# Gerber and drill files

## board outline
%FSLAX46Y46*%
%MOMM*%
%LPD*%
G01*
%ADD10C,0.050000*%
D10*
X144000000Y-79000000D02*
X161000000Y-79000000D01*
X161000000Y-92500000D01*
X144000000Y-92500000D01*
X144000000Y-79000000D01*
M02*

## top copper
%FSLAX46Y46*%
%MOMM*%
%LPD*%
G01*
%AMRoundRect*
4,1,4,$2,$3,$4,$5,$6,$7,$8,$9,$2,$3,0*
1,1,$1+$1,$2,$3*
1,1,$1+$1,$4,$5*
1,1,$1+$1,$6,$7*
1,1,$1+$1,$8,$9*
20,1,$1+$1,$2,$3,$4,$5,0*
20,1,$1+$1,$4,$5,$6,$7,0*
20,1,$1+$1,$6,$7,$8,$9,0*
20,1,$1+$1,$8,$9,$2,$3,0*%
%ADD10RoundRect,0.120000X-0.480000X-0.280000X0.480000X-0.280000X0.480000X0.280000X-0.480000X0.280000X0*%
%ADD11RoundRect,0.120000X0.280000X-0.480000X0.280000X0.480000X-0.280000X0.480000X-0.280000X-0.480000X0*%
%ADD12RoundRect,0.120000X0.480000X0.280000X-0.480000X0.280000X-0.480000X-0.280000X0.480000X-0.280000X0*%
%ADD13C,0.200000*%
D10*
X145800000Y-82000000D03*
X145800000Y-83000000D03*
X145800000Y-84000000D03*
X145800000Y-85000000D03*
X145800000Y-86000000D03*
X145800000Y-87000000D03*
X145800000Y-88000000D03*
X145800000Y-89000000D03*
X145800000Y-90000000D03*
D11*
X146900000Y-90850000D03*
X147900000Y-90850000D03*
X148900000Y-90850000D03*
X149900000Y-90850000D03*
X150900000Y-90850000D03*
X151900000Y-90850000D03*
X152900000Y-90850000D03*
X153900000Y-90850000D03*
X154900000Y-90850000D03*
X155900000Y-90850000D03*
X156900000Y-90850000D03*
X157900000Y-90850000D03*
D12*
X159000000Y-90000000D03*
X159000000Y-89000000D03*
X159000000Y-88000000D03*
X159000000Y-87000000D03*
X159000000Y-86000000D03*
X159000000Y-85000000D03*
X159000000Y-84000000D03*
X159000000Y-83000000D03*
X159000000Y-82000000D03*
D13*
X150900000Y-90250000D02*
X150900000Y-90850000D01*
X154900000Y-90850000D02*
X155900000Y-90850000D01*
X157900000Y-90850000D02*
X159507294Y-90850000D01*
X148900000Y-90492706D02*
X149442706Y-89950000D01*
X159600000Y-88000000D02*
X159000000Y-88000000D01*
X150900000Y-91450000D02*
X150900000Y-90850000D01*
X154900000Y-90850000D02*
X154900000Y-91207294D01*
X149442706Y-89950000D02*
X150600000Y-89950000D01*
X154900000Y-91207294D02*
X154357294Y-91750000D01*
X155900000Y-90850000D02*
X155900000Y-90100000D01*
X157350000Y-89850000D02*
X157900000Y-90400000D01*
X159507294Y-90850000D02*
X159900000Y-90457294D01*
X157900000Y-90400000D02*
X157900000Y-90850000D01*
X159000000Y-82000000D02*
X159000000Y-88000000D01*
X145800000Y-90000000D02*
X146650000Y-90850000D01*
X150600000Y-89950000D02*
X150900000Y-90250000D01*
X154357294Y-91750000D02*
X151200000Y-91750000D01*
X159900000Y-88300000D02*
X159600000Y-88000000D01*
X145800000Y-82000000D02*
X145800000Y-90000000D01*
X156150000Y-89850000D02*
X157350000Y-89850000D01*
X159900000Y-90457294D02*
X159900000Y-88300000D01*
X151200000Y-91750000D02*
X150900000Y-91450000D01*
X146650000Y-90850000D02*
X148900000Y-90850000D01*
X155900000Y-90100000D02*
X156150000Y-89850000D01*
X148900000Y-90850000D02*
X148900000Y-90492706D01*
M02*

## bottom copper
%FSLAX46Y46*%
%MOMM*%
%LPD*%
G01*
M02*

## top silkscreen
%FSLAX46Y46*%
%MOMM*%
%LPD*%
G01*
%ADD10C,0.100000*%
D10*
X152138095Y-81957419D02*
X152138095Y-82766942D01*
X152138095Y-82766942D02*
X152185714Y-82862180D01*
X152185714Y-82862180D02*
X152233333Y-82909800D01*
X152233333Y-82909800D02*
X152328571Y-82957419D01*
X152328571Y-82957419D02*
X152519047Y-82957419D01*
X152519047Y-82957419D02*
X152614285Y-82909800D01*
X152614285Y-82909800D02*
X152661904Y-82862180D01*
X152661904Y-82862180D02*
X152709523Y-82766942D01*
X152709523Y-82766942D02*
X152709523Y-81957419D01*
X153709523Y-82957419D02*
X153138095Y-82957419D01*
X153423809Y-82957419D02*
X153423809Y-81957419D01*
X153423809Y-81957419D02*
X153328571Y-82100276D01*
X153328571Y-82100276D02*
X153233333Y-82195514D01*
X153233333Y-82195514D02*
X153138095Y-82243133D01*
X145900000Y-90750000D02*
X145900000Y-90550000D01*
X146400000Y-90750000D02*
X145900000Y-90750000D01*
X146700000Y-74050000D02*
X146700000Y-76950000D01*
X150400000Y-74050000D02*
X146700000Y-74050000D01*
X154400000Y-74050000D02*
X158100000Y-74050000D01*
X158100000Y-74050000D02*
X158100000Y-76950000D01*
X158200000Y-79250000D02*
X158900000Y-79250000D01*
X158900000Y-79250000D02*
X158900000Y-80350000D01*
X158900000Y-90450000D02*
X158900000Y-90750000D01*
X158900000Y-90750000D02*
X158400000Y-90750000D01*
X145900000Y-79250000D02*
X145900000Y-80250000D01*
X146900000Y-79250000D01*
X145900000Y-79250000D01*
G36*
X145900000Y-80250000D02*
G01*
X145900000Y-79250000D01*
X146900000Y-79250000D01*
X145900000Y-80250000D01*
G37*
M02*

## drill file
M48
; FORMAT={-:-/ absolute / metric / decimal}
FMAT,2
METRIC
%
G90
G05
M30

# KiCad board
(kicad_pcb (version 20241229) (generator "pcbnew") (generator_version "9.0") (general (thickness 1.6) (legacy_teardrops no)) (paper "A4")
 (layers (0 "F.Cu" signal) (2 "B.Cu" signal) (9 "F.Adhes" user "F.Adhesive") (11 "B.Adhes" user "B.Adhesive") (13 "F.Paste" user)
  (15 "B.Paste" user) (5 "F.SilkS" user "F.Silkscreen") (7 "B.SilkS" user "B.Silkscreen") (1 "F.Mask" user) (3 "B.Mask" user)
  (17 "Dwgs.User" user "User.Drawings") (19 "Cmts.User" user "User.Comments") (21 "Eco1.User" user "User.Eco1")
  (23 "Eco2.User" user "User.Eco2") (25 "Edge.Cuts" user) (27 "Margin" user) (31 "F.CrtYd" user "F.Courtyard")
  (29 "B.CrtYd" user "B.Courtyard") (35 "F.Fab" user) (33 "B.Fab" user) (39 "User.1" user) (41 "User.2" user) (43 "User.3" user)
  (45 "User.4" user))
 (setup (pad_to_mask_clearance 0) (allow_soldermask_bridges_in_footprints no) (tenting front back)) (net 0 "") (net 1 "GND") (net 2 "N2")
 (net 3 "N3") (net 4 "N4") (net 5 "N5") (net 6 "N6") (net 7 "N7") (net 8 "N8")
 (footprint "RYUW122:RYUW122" (layer "F.Cu") (at 152.4 82.95)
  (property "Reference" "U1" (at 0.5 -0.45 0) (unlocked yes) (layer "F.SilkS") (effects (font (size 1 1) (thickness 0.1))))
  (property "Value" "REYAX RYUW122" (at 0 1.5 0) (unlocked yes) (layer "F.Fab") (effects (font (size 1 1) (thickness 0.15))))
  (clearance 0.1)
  (fp_line (start -6.5 7.8) (end -6.5 7.6) (stroke (width 0.1) (type default)) (layer "F.SilkS"))
  (fp_line (start -6 7.8) (end -6.5 7.8) (stroke (width 0.1) (type default)) (layer "F.SilkS"))
  (fp_line (start -5.7 -8.9) (end -5.7 -6) (stroke (width 0.1) (type default)) (layer "F.SilkS"))
  (fp_line (start -2 -8.9) (end -5.7 -8.9) (stroke (width 0.1) (type default)) (layer "F.SilkS"))
  (fp_line (start 2 -8.9) (end 5.7 -8.9) (stroke (width 0.1) (type default)) (layer "F.SilkS"))
  (fp_line (start 5.7 -8.9) (end 5.7 -6) (stroke (width 0.1) (type default)) (layer "F.SilkS"))
  (fp_line (start 5.8 -3.7) (end 6.5 -3.7) (stroke (width 0.1) (type default)) (layer "F.SilkS"))
  (fp_line (start 6.5 -3.7) (end 6.5 -2.6) (stroke (width 0.1) (type default)) (layer "F.SilkS"))
  (fp_line (start 6.5 7.5) (end 6.5 7.8) (stroke (width 0.1) (type default)) (layer "F.SilkS"))
  (fp_line (start 6.5 7.8) (end 6 7.8) (stroke (width 0.1) (type default)) (layer "F.SilkS"))
  (fp_poly (pts (xy -6.5 -3.7) (xy -6.5 -2.7) (xy -5.5 -3.7)) (stroke (width 0.1) (type solid)) (fill yes) (layer "F.SilkS"))
  (pad "1" smd roundrect (at -6.6 -0.95) (size 1.2 0.8) (layers "F.Cu" "F.Mask" "F.Paste") (roundrect_rratio 0.15) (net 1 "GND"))
  (pad "2" smd roundrect (at -6.6 0.05) (size 1.2 0.8) (layers "F.Cu" "F.Mask" "F.Paste") (roundrect_rratio 0.15) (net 1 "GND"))
  (pad "3" smd roundrect (at -6.6 1.05) (size 1.2 0.8) (layers "F.Cu" "F.Mask" "F.Paste") (roundrect_rratio 0.15) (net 1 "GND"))
  (pad "4" smd roundrect (at -6.6 2.05) (size 1.2 0.8) (layers "F.Cu" "F.Mask" "F.Paste") (roundrect_rratio 0.15) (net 1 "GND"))
  (pad "5" smd roundrect (at -6.6 3.05) (size 1.2 0.8) (layers "F.Cu" "F.Mask" "F.Paste") (roundrect_rratio 0.15) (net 1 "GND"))
  (pad "6" smd roundrect (at -6.6 4.05) (size 1.2 0.8) (layers "F.Cu" "F.Mask" "F.Paste") (roundrect_rratio 0.15) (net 1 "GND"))
  (pad "7" smd roundrect (at -6.6 5.05) (size 1.2 0.8) (layers "F.Cu" "F.Mask" "F.Paste") (roundrect_rratio 0.15) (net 1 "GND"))
  (pad "8" smd roundrect (at -6.6 6.05) (size 1.2 0.8) (layers "F.Cu" "F.Mask" "F.Paste") (roundrect_rratio 0.15) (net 1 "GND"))
  (pad "9" smd roundrect (at -6.6 7.05) (size 1.2 0.8) (layers "F.Cu" "F.Mask" "F.Paste") (roundrect_rratio 0.15) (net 1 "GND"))
  (pad "10" smd roundrect (at -5.5 7.9 90) (size 1.2 0.8) (layers "F.Cu" "F.Mask" "F.Paste") (roundrect_rratio 0.15) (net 1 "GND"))
  (pad "11" smd roundrect (at -4.5 7.9 90) (size 1.2 0.8) (layers "F.Cu" "F.Mask" "F.Paste") (roundrect_rratio 0.15) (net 1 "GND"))
  (pad "12" smd roundrect (at -3.5 7.9 90) (size 1.2 0.8) (layers "F.Cu" "F.Mask" "F.Paste") (roundrect_rratio 0.15) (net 1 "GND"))
  (pad "13" smd roundrect (at -2.5 7.9 90) (size 1.2 0.8) (layers "F.Cu" "F.Mask" "F.Paste") (roundrect_rratio 0.15) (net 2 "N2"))
  (pad "14" smd roundrect (at -1.5 7.9 90) (size 1.2 0.8) (layers "F.Cu" "F.Mask" "F.Paste") (roundrect_rratio 0.15) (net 1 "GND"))
  (pad "15" smd roundrect (at -0.5 7.9 90) (size 1.2 0.8) (layers "F.Cu" "F.Mask" "F.Paste") (roundrect_rratio 0.15) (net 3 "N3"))
  (pad "16" smd roundrect (at 0.5 7.9 90) (size 1.2 0.8) (layers "F.Cu" "F.Mask" "F.Paste") (roundrect_rratio 0.15) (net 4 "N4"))
  (pad "17" smd roundrect (at 1.5 7.9 90) (size 1.2 0.8) (layers "F.Cu" "F.Mask" "F.Paste") (roundrect_rratio 0.15) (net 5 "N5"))
  (pad "18" smd roundrect (at 2.5 7.9 90) (size 1.2 0.8) (layers "F.Cu" "F.Mask" "F.Paste") (roundrect_rratio 0.15) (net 1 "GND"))
  (pad "19" smd roundrect (at 3.5 7.9 90) (size 1.2 0.8) (layers "F.Cu" "F.Mask" "F.Paste") (roundrect_rratio 0.15) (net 1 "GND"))
  (pad "20" smd roundrect (at 4.5 7.9 90) (size 1.2 0.8) (layers "F.Cu" "F.Mask" "F.Paste") (roundrect_rratio 0.15) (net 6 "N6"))
  (pad "21" smd roundrect (at 5.5 7.9 90) (size 1.2 0.8) (layers "F.Cu" "F.Mask" "F.Paste") (roundrect_rratio 0.15) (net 1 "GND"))
  (pad "22" smd roundrect (at 6.6 7.05 180) (size 1.2 0.8) (layers "F.Cu" "F.Mask" "F.Paste") (roundrect_rratio 0.15) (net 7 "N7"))
  (pad "23" smd roundrect (at 6.6 6.05 180) (size 1.2 0.8) (layers "F.Cu" "F.Mask" "F.Paste") (roundrect_rratio 0.15) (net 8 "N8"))
  (pad "24" smd roundrect (at 6.6 5.05 180) (size 1.2 0.8) (layers "F.Cu" "F.Mask" "F.Paste") (roundrect_rratio 0.15) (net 1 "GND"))
  (pad "25" smd roundrect (at 6.6 4.05 180) (size 1.2 0.8) (layers "F.Cu" "F.Mask" "F.Paste") (roundrect_rratio 0.15) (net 1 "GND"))
  (pad "26" smd roundrect (at 6.6 3.05 180) (size 1.2 0.8) (layers "F.Cu" "F.Mask" "F.Paste") (roundrect_rratio 0.15) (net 1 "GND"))
  (pad "27" smd roundrect (at 6.6 2.05 180) (size 1.2 0.8) (layers "F.Cu" "F.Mask" "F.Paste") (roundrect_rratio 0.15) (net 1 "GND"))
  (pad "28" smd roundrect (at 6.6 1.05 180) (size 1.2 0.8) (layers "F.Cu" "F.Mask" "F.Paste") (roundrect_rratio 0.15) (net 1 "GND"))
  (pad "29" smd roundrect (at 6.6 0.05 180) (size 1.2 0.8) (layers "F.Cu" "F.Mask" "F.Paste") (roundrect_rratio 0.15) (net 1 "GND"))
  (pad "30" smd roundrect (at 6.6 -0.95 180) (size 1.2 0.8) (layers "F.Cu" "F.Mask" "F.Paste") (roundrect_rratio 0.15) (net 1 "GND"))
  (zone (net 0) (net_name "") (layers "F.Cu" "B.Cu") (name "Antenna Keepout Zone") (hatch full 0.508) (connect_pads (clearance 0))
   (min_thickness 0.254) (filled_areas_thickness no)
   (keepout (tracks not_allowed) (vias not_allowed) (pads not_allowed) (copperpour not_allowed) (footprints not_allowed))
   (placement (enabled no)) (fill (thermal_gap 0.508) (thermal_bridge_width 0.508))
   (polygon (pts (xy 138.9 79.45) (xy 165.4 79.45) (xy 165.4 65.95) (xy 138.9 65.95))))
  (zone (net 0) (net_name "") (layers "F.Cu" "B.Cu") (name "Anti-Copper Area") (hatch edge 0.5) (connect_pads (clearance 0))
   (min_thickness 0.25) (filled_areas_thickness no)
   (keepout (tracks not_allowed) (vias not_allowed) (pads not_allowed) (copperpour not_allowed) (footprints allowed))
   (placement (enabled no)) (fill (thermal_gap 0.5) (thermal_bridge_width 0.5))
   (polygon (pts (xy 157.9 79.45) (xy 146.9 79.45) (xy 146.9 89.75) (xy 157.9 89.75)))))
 (gr_rect (start 144 79) (end 161 92.5) (stroke (width 0.05) (type default)) (fill no) (layer "Edge.Cuts"))
 (segment (start 150.9 90.25) (end 150.9 90.85) (width 0.2) (layer "F.Cu") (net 1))
 (segment (start 154.9 90.85) (end 155.9 90.85) (width 0.2) (layer "F.Cu") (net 1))
 (segment (start 157.9 90.85) (end 159.507294 90.85) (width 0.2) (layer "F.Cu") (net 1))
 (segment (start 148.9 90.492706) (end 149.442706 89.95) (width 0.2) (layer "F.Cu") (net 1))
 (segment (start 159.6 88) (end 159 88) (width 0.2) (layer "F.Cu") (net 1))
 (segment (start 150.9 91.45) (end 150.9 90.85) (width 0.2) (layer "F.Cu") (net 1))
 (segment (start 154.9 90.85) (end 154.9 91.207294) (width 0.2) (layer "F.Cu") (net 1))
 (segment (start 149.442706 89.95) (end 150.6 89.95) (width 0.2) (layer "F.Cu") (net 1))
 (segment (start 154.9 91.207294) (end 154.357294 91.75) (width 0.2) (layer "F.Cu") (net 1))
 (segment (start 155.9 90.85) (end 155.9 90.1) (width 0.2) (layer "F.Cu") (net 1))
 (segment (start 157.35 89.85) (end 157.9 90.4) (width 0.2) (layer "F.Cu") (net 1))
 (segment (start 159.507294 90.85) (end 159.9 90.457294) (width 0.2) (layer "F.Cu") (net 1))
 (segment (start 157.9 90.4) (end 157.9 90.85) (width 0.2) (layer "F.Cu") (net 1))
 (segment (start 159 82) (end 159 88) (width 0.2) (layer "F.Cu") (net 1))
 (segment (start 145.8 90) (end 146.65 90.85) (width 0.2) (layer "F.Cu") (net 1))
 (segment (start 150.6 89.95) (end 150.9 90.25) (width 0.2) (layer "F.Cu") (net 1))
 (segment (start 154.357294 91.75) (end 151.2 91.75) (width 0.2) (layer "F.Cu") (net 1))
 (segment (start 159.9 88.3) (end 159.6 88) (width 0.2) (layer "F.Cu") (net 1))
 (segment (start 145.8 82) (end 145.8 90) (width 0.2) (layer "F.Cu") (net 1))
 (segment (start 156.15 89.85) (end 157.35 89.85) (width 0.2) (layer "F.Cu") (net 1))
 (segment (start 159.9 90.457294) (end 159.9 88.3) (width 0.2) (layer "F.Cu") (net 1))
 (segment (start 151.2 91.75) (end 150.9 91.45) (width 0.2) (layer "F.Cu") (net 1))
 (segment (start 146.65 90.85) (end 148.9 90.85) (width 0.2) (layer "F.Cu") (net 1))
 (segment (start 155.9 90.1) (end 156.15 89.85) (width 0.2) (layer "F.Cu") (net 1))
 (segment (start 148.9 90.85) (end 148.9 90.492706) (width 0.2) (layer "F.Cu") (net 1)))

